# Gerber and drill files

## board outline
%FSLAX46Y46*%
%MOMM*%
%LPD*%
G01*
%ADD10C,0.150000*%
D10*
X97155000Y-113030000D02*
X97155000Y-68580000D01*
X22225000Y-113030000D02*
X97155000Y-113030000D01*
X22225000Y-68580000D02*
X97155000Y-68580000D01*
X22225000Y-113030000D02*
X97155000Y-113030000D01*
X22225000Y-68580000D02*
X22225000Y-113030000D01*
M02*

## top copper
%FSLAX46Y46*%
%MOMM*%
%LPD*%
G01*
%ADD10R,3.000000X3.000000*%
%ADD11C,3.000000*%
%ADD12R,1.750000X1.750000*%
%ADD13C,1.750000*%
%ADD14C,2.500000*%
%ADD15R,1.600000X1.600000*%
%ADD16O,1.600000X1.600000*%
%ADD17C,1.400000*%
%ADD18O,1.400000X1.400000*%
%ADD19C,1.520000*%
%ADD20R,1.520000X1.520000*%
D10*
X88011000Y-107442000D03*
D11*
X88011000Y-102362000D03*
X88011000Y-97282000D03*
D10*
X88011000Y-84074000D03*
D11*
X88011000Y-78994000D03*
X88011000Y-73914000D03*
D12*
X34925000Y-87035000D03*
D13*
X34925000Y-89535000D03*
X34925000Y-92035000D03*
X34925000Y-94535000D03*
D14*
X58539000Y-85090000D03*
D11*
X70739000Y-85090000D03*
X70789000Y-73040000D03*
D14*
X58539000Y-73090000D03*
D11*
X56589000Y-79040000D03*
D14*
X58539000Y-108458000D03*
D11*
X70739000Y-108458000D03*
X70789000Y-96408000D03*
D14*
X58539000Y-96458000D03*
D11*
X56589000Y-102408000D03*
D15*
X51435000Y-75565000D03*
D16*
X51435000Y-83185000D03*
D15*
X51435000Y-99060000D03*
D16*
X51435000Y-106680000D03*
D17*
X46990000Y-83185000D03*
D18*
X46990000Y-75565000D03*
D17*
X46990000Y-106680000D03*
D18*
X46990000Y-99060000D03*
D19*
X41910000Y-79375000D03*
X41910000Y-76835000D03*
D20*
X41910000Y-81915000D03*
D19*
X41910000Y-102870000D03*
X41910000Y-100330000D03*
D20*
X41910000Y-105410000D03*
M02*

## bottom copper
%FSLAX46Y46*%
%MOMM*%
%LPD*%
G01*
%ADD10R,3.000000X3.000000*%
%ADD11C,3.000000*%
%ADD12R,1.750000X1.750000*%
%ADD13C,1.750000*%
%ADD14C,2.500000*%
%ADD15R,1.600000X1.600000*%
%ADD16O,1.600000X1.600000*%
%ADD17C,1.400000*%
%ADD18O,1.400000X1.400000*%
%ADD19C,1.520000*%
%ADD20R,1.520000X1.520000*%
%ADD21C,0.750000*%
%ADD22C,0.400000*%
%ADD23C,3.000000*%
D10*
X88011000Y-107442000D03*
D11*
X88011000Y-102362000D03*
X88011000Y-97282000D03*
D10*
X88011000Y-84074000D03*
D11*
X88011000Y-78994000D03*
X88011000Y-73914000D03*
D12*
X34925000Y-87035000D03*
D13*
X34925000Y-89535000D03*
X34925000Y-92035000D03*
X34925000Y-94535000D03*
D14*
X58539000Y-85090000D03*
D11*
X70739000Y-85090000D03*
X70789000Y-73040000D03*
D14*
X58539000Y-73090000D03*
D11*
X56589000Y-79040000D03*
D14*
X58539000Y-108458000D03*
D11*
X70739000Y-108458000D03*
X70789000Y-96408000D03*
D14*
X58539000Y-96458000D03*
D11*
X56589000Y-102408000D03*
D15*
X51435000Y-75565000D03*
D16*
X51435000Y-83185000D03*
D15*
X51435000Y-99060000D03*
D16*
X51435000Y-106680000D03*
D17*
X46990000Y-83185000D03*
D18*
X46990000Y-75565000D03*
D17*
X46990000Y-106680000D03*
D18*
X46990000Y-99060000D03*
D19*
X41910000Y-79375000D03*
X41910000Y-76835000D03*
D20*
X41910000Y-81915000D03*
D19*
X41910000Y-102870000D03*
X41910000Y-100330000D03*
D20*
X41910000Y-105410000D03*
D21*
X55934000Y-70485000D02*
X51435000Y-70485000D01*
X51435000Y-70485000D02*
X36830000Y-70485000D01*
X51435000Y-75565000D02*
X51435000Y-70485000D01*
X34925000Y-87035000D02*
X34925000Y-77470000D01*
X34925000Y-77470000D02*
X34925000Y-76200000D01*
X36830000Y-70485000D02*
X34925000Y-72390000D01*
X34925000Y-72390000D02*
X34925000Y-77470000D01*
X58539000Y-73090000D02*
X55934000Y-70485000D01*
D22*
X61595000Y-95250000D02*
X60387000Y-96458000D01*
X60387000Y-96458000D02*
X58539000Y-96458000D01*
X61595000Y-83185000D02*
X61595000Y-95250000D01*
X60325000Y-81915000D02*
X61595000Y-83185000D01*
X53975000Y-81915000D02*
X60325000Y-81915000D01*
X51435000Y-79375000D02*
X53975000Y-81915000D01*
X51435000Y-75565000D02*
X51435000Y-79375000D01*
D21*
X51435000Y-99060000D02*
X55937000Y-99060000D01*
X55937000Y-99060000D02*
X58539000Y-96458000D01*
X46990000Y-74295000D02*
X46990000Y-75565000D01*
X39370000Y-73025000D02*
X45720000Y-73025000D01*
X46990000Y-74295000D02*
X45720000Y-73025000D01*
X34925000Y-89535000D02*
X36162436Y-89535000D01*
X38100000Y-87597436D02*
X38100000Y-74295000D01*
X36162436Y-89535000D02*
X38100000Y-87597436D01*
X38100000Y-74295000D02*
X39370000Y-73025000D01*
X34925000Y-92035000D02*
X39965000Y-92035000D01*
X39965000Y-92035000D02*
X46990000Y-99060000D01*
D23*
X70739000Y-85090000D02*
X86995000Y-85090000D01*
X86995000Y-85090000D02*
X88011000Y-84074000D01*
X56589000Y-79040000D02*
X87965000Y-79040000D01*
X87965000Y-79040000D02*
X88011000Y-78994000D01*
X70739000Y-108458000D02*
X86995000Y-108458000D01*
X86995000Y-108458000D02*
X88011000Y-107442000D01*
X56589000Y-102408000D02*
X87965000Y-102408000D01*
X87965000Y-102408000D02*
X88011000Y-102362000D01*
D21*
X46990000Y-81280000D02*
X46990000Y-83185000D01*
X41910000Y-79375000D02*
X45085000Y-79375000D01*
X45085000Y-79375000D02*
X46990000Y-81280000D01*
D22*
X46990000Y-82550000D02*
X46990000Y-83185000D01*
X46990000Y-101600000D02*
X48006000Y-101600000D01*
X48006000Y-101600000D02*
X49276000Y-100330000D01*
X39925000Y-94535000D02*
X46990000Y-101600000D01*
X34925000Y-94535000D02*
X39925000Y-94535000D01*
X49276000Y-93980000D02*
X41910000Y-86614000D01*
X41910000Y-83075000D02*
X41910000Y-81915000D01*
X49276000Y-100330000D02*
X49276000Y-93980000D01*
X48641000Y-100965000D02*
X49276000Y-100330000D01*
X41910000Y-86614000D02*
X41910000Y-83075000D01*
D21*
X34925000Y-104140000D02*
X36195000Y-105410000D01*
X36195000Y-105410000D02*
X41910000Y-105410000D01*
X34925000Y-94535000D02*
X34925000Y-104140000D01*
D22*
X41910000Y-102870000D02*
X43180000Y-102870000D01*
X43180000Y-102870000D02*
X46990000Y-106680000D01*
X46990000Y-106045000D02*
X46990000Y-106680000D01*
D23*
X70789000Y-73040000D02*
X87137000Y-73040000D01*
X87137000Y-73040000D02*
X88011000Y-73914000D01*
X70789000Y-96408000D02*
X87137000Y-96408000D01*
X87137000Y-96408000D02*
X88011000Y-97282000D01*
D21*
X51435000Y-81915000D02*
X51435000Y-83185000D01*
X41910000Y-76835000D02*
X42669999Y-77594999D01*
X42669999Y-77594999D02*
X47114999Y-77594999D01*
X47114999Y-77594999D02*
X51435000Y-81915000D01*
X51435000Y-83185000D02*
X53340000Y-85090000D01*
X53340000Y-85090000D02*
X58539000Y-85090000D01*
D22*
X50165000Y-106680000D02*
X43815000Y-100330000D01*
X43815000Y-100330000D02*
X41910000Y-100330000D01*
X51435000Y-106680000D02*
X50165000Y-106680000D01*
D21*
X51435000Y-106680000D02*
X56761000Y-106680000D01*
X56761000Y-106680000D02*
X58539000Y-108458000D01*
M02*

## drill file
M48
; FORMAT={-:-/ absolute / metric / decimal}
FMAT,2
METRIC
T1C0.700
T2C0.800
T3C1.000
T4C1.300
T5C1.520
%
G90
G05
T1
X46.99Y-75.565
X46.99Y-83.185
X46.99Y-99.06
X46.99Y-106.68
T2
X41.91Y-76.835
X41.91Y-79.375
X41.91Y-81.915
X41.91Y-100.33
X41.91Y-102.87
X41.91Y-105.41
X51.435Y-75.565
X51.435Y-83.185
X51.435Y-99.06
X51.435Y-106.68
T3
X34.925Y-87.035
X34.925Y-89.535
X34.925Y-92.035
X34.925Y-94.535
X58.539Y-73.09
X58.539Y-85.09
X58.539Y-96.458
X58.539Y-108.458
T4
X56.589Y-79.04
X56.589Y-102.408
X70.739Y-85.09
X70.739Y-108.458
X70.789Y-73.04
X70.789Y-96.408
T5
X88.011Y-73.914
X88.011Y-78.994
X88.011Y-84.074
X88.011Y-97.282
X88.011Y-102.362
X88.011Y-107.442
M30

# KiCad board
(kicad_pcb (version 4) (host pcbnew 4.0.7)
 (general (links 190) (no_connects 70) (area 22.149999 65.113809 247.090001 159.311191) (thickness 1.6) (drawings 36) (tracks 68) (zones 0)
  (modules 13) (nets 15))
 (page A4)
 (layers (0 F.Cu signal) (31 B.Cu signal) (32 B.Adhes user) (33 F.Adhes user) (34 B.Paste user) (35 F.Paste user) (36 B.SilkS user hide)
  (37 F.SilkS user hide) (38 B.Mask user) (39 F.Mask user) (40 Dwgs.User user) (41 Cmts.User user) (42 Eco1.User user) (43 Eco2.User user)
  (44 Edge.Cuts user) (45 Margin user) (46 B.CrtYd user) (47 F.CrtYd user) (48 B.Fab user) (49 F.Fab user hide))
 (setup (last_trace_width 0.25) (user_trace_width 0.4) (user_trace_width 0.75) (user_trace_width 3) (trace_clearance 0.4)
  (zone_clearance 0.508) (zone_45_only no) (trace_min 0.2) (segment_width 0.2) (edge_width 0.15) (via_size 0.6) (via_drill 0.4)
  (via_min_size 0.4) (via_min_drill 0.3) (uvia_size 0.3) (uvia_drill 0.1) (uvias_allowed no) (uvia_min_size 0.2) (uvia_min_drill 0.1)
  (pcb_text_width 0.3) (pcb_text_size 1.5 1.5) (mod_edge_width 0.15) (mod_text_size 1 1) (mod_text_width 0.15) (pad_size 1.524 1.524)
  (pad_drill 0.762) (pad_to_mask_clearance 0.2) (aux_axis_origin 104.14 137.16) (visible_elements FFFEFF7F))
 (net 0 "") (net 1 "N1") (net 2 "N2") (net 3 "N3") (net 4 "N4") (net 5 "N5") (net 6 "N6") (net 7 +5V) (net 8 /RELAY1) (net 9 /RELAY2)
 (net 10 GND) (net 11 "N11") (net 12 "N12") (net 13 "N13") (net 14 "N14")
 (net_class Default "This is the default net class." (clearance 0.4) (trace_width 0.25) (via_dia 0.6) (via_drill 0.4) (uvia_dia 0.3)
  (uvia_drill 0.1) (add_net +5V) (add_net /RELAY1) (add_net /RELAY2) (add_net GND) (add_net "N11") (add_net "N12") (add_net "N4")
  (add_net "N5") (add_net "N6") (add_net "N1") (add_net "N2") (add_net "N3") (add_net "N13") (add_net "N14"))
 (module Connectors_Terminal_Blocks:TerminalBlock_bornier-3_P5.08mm (layer F.Cu) (at 88.011 107.442 90)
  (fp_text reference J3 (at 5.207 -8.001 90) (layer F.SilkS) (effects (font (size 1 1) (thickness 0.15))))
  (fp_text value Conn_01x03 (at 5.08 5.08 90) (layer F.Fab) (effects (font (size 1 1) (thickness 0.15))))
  (pad 1 thru_hole rect (at 0 0 90) (size 3 3) (drill 1.52) (layers *.Cu *.Mask) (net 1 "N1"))
  (pad 2 thru_hole circle (at 5.08 0 90) (size 3 3) (drill 1.52) (layers *.Cu *.Mask) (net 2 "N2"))
  (pad 3 thru_hole circle (at 10.16 0 90) (size 3 3) (drill 1.52) (layers *.Cu *.Mask) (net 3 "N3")))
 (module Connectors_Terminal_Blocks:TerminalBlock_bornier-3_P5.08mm (layer F.Cu) (at 88.011 84.074 90)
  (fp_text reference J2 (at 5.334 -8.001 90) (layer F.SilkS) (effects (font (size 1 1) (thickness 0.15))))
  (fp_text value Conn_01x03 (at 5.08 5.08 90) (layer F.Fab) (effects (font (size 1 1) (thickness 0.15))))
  (pad 1 thru_hole rect (at 0 0 90) (size 3 3) (drill 1.52) (layers *.Cu *.Mask) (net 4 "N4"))
  (pad 2 thru_hole circle (at 5.08 0 90) (size 3 3) (drill 1.52) (layers *.Cu *.Mask) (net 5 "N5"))
  (pad 3 thru_hole circle (at 10.16 0 90) (size 3 3) (drill 1.52) (layers *.Cu *.Mask) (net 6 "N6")))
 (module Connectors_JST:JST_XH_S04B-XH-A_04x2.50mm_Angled (layer F.Cu) (at 34.925 87.035 270)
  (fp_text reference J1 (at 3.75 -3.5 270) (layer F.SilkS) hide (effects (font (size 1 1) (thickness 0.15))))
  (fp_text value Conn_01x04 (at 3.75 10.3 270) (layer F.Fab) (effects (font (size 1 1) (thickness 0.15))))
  (pad 1 thru_hole rect (at 0 0 270) (size 1.75 1.75) (drill 1) (layers *.Cu *.Mask F.SilkS) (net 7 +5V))
  (pad 2 thru_hole circle (at 2.5 0 270) (size 1.75 1.75) (drill 1) (layers *.Cu *.Mask F.SilkS) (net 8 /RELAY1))
  (pad 3 thru_hole circle (at 5 0 270) (size 1.75 1.75) (drill 1) (layers *.Cu *.Mask F.SilkS) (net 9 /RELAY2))
  (pad 4 thru_hole circle (at 7.5 0 270) (size 1.75 1.75) (drill 1) (layers *.Cu *.Mask F.SilkS) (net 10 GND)))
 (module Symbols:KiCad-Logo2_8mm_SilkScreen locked (layer B.Cu) (at 79.375 102.235 270)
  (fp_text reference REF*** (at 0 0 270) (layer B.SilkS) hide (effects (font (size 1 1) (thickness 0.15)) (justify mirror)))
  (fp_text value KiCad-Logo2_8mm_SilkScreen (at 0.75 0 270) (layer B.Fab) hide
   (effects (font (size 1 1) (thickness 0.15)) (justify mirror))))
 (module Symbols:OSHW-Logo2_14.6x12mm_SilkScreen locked (layer B.Cu) (at 78.74 78.74 270)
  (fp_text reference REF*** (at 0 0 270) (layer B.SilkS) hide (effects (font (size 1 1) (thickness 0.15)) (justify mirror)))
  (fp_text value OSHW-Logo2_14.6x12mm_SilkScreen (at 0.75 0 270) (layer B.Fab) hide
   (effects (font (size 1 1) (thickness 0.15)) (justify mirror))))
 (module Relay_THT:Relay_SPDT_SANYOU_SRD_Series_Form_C (layer F.Cu) (at 56.589 79.04)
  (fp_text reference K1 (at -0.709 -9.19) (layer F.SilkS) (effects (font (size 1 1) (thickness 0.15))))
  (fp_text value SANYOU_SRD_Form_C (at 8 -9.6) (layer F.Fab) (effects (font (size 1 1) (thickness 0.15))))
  (pad 2 thru_hole circle (at 1.95 6.05 90) (size 2.5 2.5) (drill 1) (layers *.Cu *.Mask) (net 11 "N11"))
  (pad 3 thru_hole circle (at 14.15 6.05 90) (size 3 3) (drill 1.3) (layers *.Cu *.Mask) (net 4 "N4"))
  (pad 4 thru_hole circle (at 14.2 -6 90) (size 3 3) (drill 1.3) (layers *.Cu *.Mask) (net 6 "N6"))
  (pad 5 thru_hole circle (at 1.95 -5.95 90) (size 2.5 2.5) (drill 1) (layers *.Cu *.Mask) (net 7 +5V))
  (pad 1 thru_hole circle (at 0 0 90) (size 3 3) (drill 1.3) (layers *.Cu *.Mask) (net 5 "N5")))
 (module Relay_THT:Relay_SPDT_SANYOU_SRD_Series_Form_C (layer F.Cu) (at 56.589 102.408)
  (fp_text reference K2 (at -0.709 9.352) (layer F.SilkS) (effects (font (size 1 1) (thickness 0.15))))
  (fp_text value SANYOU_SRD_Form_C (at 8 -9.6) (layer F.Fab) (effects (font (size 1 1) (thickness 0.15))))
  (pad 2 thru_hole circle (at 1.95 6.05 90) (size 2.5 2.5) (drill 1) (layers *.Cu *.Mask) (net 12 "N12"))
  (pad 3 thru_hole circle (at 14.15 6.05 90) (size 3 3) (drill 1.3) (layers *.Cu *.Mask) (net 1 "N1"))
  (pad 4 thru_hole circle (at 14.2 -6 90) (size 3 3) (drill 1.3) (layers *.Cu *.Mask) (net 3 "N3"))
  (pad 5 thru_hole circle (at 1.95 -5.95 90) (size 2.5 2.5) (drill 1) (layers *.Cu *.Mask) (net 7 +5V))
  (pad 1 thru_hole circle (at 0 0 90) (size 3 3) (drill 1.3) (layers *.Cu *.Mask) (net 2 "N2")))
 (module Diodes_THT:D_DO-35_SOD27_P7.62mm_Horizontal (layer F.Cu) (at 51.435 75.565 270)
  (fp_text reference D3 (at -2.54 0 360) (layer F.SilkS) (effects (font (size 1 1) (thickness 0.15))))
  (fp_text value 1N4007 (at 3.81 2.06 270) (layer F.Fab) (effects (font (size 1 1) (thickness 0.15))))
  (pad 1 thru_hole rect (at 0 0 270) (size 1.6 1.6) (drill 0.8) (layers *.Cu *.Mask) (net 7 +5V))
  (pad 2 thru_hole oval (at 7.62 0 270) (size 1.6 1.6) (drill 0.8) (layers *.Cu *.Mask) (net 11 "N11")))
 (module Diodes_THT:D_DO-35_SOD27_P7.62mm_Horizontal (layer F.Cu) (at 51.435 99.06 270)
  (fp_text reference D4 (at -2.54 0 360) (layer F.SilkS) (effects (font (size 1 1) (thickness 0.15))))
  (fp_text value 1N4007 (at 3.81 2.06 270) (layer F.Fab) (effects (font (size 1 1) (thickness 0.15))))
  (pad 1 thru_hole rect (at 0 0 270) (size 1.6 1.6) (drill 0.8) (layers *.Cu *.Mask) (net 7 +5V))
  (pad 2 thru_hole oval (at 7.62 0 270) (size 1.6 1.6) (drill 0.8) (layers *.Cu *.Mask) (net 12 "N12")))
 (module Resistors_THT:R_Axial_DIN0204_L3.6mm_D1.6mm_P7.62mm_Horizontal (layer F.Cu) (at 46.99 83.185 90)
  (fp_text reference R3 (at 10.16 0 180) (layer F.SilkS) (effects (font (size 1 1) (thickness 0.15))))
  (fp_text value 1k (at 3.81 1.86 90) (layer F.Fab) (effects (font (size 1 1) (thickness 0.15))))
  (pad 1 thru_hole circle (at 0 0 90) (size 1.4 1.4) (drill 0.7) (layers *.Cu *.Mask) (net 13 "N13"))
  (pad 2 thru_hole oval (at 7.62 0 90) (size 1.4 1.4) (drill 0.7) (layers *.Cu *.Mask) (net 8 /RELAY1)))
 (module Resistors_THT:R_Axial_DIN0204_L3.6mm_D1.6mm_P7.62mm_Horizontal (layer F.Cu) (at 46.99 106.68 90)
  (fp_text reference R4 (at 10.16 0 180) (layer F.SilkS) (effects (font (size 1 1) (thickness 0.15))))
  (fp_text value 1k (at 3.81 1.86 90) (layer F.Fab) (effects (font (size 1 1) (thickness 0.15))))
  (pad 1 thru_hole circle (at 0 0 90) (size 1.4 1.4) (drill 0.7) (layers *.Cu *.Mask) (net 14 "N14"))
  (pad 2 thru_hole oval (at 7.62 0 90) (size 1.4 1.4) (drill 0.7) (layers *.Cu *.Mask) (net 9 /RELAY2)))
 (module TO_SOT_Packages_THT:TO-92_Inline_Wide (layer F.Cu) (at 41.91 81.915 90)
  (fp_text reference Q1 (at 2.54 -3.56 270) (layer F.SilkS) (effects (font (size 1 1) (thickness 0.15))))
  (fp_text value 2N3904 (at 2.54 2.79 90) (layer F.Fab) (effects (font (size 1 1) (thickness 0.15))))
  (pad 2 thru_hole circle (at 2.54 0 180) (size 1.52 1.52) (drill 0.8) (layers *.Cu *.Mask) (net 13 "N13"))
  (pad 3 thru_hole circle (at 5.08 0 180) (size 1.52 1.52) (drill 0.8) (layers *.Cu *.Mask) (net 11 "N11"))
  (pad 1 thru_hole rect (at 0 0 180) (size 1.52 1.52) (drill 0.8) (layers *.Cu *.Mask) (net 10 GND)))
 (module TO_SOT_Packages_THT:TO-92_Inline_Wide (layer F.Cu) (at 41.91 105.41 90)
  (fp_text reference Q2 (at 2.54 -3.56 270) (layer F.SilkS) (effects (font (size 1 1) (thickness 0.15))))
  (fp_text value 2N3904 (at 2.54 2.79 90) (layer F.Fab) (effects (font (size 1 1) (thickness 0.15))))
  (pad 2 thru_hole circle (at 2.54 0 180) (size 1.52 1.52) (drill 0.8) (layers *.Cu *.Mask) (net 14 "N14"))
  (pad 3 thru_hole circle (at 5.08 0 180) (size 1.52 1.52) (drill 0.8) (layers *.Cu *.Mask) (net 12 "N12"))
  (pad 1 thru_hole rect (at 0 0 180) (size 1.52 1.52) (drill 0.8) (layers *.Cu *.Mask) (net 10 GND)))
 (gr_line (start 97.155 113.03) (end 97.155 68.58) (layer Edge.Cuts) (width 0.15))
 (gr_line (start 22.225 113.03) (end 97.155 113.03) (layer Edge.Cuts) (width 0.15))
 (gr_line (start 22.225 68.58) (end 97.155 68.58) (layer Edge.Cuts) (width 0.15))
 (gr_line (start 22.225 113.03) (end 97.155 113.03) (layer Edge.Cuts) (width 0.15))
 (gr_line (start 22.225 68.58) (end 22.225 113.03) (layer Edge.Cuts) (width 0.15))
 (segment (start 55.934 70.485) (end 51.435 70.485) (width 0.75) (layer B.Cu) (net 7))
 (segment (start 51.435 70.485) (end 36.83 70.485) (width 0.75) (layer B.Cu) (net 7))
 (segment (start 51.435 75.565) (end 51.435 70.485) (width 0.75) (layer B.Cu) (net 7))
 (segment (start 34.925 87.035) (end 34.925 77.47) (width 0.75) (layer B.Cu) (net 7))
 (segment (start 34.925 77.47) (end 34.925 76.2) (width 0.75) (layer B.Cu) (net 7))
 (segment (start 36.83 70.485) (end 34.925 72.39) (width 0.75) (layer B.Cu) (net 7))
 (segment (start 34.925 72.39) (end 34.925 77.47) (width 0.75) (layer B.Cu) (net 7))
 (segment (start 58.539 73.09) (end 55.934 70.485) (width 0.75) (layer B.Cu) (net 7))
 (segment (start 61.595 95.25) (end 60.387 96.458) (width 0.4) (layer B.Cu) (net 7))
 (segment (start 60.387 96.458) (end 58.539 96.458) (width 0.4) (layer B.Cu) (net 7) (status 20))
 (segment (start 61.595 83.185) (end 61.595 95.25) (width 0.4) (layer B.Cu) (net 7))
 (segment (start 60.325 81.915) (end 61.595 83.185) (width 0.4) (layer B.Cu) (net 7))
 (segment (start 53.975 81.915) (end 60.325 81.915) (width 0.4) (layer B.Cu) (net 7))
 (segment (start 51.435 79.375) (end 53.975 81.915) (width 0.4) (layer B.Cu) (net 7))
 (segment (start 51.435 75.565) (end 51.435 79.375) (width 0.4) (layer B.Cu) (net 7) (status 10))
 (segment (start 51.435 99.06) (end 55.937 99.06) (width 0.75) (layer B.Cu) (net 7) (status 10))
 (segment (start 55.937 99.06) (end 58.539 96.458) (width 0.75) (layer B.Cu) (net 7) (status 20))
 (segment (start 46.99 74.295) (end 46.99 75.565) (width 0.75) (layer B.Cu) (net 8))
 (segment (start 39.37 73.025) (end 45.72 73.025) (width 0.75) (layer B.Cu) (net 8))
 (segment (start 46.99 74.295) (end 45.72 73.025) (width 0.75) (layer B.Cu) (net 8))
 (segment (start 34.925 89.535) (end 36.162436 89.535) (width 0.75) (layer B.Cu) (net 8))
 (segment (start 38.1 87.597436) (end 38.1 74.295) (width 0.75) (layer B.Cu) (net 8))
 (segment (start 36.162436 89.535) (end 38.1 87.597436) (width 0.75) (layer B.Cu) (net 8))
 (segment (start 38.1 74.295) (end 39.37 73.025) (width 0.75) (layer B.Cu) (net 8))
 (segment (start 34.925 92.035) (end 39.965 92.035) (width 0.75) (layer B.Cu) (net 9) (status 10))
 (segment (start 39.965 92.035) (end 46.99 99.06) (width 0.75) (layer B.Cu) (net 9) (status 20))
 (segment (start 70.739 85.09) (end 86.995 85.09) (width 3) (layer B.Cu) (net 4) (status 30))
 (segment (start 86.995 85.09) (end 88.011 84.074) (width 3) (layer B.Cu) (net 4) (status 30))
 (segment (start 56.589 79.04) (end 87.965 79.04) (width 3) (layer B.Cu) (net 5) (status 30))
 (segment (start 87.965 79.04) (end 88.011 78.994) (width 3) (layer B.Cu) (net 5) (status 30))
 (segment (start 70.739 108.458) (end 86.995 108.458) (width 3) (layer B.Cu) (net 1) (status 30))
 (segment (start 86.995 108.458) (end 88.011 107.442) (width 3) (layer B.Cu) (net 1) (status 30))
 (segment (start 56.589 102.408) (end 87.965 102.408) (width 3) (layer B.Cu) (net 2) (status 30))
 (segment (start 87.965 102.408) (end 88.011 102.362) (width 3) (layer B.Cu) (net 2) (status 30))
 (segment (start 46.99 81.28) (end 46.99 83.185) (width 0.75) (layer B.Cu) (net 13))
 (segment (start 41.91 79.375) (end 45.085 79.375) (width 0.75) (layer B.Cu) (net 13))
 (segment (start 45.085 79.375) (end 46.99 81.28) (width 0.75) (layer B.Cu) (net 13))
 (segment (start 46.99 82.55) (end 46.99 83.185) (width 0.4) (layer B.Cu) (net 13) (status 30))
 (segment (start 46.99 101.6) (end 48.006 101.6) (width 0.4) (layer B.Cu) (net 10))
 (segment (start 48.006 101.6) (end 49.276 100.33) (width 0.4) (layer B.Cu) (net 10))
 (segment (start 39.925 94.535) (end 46.99 101.6) (width 0.4) (layer B.Cu) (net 10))
 (segment (start 34.925 94.535) (end 39.925 94.535) (width 0.4) (layer B.Cu) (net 10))
 (segment (start 49.276 93.98) (end 41.91 86.614) (width 0.4) (layer B.Cu) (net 10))
 (segment (start 41.91 83.075) (end 41.91 81.915) (width 0.4) (layer B.Cu) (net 10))
 (segment (start 49.276 100.33) (end 49.276 93.98) (width 0.4) (layer B.Cu) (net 10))
 (segment (start 48.641 100.965) (end 49.276 100.33) (width 0.4) (layer B.Cu) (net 10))
 (segment (start 41.91 86.614) (end 41.91 83.075) (width 0.4) (layer B.Cu) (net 10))
 (segment (start 34.925 104.14) (end 36.195 105.41) (width 0.75) (layer B.Cu) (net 10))
 (segment (start 36.195 105.41) (end 41.91 105.41) (width 0.75) (layer B.Cu) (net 10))
 (segment (start 34.925 94.535) (end 34.925 104.14) (width 0.75) (layer B.Cu) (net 10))
 (segment (start 41.91 102.87) (end 43.18 102.87) (width 0.4) (layer B.Cu) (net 14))
 (segment (start 43.18 102.87) (end 46.99 106.68) (width 0.4) (layer B.Cu) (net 14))
 (segment (start 46.99 106.045) (end 46.99 106.68) (width 0.4) (layer B.Cu) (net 14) (status 30))
 (segment (start 70.789 73.04) (end 87.137 73.04) (width 3) (layer B.Cu) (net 6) (status 30))
 (segment (start 87.137 73.04) (end 88.011 73.914) (width 3) (layer B.Cu) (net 6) (status 30))
 (segment (start 70.789 96.408) (end 87.137 96.408) (width 3) (layer B.Cu) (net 3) (status 30))
 (segment (start 87.137 96.408) (end 88.011 97.282) (width 3) (layer B.Cu) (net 3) (status 30))
 (segment (start 51.435 81.915) (end 51.435 83.185) (width 0.75) (layer B.Cu) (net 11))
 (segment (start 41.91 76.835) (end 42.669999 77.594999) (width 0.75) (layer B.Cu) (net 11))
 (segment (start 42.669999 77.594999) (end 47.114999 77.594999) (width 0.75) (layer B.Cu) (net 11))
 (segment (start 47.114999 77.594999) (end 51.435 81.915) (width 0.75) (layer B.Cu) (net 11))
 (segment (start 51.435 83.185) (end 53.34 85.09) (width 0.75) (layer B.Cu) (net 11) (status 10))
 (segment (start 53.34 85.09) (end 58.539 85.09) (width 0.75) (layer B.Cu) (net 11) (status 20))
 (segment (start 50.165 106.68) (end 43.815 100.33) (width 0.4) (layer B.Cu) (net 12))
 (segment (start 43.815 100.33) (end 41.91 100.33) (width 0.4) (layer B.Cu) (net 12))
 (segment (start 51.435 106.68) (end 50.165 106.68) (width 0.4) (layer B.Cu) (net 12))
 (segment (start 51.435 106.68) (end 56.761 106.68) (width 0.75) (layer B.Cu) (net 12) (status 10))
 (segment (start 56.761 106.68) (end 58.539 108.458) (width 0.75) (layer B.Cu) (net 12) (status 20)))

